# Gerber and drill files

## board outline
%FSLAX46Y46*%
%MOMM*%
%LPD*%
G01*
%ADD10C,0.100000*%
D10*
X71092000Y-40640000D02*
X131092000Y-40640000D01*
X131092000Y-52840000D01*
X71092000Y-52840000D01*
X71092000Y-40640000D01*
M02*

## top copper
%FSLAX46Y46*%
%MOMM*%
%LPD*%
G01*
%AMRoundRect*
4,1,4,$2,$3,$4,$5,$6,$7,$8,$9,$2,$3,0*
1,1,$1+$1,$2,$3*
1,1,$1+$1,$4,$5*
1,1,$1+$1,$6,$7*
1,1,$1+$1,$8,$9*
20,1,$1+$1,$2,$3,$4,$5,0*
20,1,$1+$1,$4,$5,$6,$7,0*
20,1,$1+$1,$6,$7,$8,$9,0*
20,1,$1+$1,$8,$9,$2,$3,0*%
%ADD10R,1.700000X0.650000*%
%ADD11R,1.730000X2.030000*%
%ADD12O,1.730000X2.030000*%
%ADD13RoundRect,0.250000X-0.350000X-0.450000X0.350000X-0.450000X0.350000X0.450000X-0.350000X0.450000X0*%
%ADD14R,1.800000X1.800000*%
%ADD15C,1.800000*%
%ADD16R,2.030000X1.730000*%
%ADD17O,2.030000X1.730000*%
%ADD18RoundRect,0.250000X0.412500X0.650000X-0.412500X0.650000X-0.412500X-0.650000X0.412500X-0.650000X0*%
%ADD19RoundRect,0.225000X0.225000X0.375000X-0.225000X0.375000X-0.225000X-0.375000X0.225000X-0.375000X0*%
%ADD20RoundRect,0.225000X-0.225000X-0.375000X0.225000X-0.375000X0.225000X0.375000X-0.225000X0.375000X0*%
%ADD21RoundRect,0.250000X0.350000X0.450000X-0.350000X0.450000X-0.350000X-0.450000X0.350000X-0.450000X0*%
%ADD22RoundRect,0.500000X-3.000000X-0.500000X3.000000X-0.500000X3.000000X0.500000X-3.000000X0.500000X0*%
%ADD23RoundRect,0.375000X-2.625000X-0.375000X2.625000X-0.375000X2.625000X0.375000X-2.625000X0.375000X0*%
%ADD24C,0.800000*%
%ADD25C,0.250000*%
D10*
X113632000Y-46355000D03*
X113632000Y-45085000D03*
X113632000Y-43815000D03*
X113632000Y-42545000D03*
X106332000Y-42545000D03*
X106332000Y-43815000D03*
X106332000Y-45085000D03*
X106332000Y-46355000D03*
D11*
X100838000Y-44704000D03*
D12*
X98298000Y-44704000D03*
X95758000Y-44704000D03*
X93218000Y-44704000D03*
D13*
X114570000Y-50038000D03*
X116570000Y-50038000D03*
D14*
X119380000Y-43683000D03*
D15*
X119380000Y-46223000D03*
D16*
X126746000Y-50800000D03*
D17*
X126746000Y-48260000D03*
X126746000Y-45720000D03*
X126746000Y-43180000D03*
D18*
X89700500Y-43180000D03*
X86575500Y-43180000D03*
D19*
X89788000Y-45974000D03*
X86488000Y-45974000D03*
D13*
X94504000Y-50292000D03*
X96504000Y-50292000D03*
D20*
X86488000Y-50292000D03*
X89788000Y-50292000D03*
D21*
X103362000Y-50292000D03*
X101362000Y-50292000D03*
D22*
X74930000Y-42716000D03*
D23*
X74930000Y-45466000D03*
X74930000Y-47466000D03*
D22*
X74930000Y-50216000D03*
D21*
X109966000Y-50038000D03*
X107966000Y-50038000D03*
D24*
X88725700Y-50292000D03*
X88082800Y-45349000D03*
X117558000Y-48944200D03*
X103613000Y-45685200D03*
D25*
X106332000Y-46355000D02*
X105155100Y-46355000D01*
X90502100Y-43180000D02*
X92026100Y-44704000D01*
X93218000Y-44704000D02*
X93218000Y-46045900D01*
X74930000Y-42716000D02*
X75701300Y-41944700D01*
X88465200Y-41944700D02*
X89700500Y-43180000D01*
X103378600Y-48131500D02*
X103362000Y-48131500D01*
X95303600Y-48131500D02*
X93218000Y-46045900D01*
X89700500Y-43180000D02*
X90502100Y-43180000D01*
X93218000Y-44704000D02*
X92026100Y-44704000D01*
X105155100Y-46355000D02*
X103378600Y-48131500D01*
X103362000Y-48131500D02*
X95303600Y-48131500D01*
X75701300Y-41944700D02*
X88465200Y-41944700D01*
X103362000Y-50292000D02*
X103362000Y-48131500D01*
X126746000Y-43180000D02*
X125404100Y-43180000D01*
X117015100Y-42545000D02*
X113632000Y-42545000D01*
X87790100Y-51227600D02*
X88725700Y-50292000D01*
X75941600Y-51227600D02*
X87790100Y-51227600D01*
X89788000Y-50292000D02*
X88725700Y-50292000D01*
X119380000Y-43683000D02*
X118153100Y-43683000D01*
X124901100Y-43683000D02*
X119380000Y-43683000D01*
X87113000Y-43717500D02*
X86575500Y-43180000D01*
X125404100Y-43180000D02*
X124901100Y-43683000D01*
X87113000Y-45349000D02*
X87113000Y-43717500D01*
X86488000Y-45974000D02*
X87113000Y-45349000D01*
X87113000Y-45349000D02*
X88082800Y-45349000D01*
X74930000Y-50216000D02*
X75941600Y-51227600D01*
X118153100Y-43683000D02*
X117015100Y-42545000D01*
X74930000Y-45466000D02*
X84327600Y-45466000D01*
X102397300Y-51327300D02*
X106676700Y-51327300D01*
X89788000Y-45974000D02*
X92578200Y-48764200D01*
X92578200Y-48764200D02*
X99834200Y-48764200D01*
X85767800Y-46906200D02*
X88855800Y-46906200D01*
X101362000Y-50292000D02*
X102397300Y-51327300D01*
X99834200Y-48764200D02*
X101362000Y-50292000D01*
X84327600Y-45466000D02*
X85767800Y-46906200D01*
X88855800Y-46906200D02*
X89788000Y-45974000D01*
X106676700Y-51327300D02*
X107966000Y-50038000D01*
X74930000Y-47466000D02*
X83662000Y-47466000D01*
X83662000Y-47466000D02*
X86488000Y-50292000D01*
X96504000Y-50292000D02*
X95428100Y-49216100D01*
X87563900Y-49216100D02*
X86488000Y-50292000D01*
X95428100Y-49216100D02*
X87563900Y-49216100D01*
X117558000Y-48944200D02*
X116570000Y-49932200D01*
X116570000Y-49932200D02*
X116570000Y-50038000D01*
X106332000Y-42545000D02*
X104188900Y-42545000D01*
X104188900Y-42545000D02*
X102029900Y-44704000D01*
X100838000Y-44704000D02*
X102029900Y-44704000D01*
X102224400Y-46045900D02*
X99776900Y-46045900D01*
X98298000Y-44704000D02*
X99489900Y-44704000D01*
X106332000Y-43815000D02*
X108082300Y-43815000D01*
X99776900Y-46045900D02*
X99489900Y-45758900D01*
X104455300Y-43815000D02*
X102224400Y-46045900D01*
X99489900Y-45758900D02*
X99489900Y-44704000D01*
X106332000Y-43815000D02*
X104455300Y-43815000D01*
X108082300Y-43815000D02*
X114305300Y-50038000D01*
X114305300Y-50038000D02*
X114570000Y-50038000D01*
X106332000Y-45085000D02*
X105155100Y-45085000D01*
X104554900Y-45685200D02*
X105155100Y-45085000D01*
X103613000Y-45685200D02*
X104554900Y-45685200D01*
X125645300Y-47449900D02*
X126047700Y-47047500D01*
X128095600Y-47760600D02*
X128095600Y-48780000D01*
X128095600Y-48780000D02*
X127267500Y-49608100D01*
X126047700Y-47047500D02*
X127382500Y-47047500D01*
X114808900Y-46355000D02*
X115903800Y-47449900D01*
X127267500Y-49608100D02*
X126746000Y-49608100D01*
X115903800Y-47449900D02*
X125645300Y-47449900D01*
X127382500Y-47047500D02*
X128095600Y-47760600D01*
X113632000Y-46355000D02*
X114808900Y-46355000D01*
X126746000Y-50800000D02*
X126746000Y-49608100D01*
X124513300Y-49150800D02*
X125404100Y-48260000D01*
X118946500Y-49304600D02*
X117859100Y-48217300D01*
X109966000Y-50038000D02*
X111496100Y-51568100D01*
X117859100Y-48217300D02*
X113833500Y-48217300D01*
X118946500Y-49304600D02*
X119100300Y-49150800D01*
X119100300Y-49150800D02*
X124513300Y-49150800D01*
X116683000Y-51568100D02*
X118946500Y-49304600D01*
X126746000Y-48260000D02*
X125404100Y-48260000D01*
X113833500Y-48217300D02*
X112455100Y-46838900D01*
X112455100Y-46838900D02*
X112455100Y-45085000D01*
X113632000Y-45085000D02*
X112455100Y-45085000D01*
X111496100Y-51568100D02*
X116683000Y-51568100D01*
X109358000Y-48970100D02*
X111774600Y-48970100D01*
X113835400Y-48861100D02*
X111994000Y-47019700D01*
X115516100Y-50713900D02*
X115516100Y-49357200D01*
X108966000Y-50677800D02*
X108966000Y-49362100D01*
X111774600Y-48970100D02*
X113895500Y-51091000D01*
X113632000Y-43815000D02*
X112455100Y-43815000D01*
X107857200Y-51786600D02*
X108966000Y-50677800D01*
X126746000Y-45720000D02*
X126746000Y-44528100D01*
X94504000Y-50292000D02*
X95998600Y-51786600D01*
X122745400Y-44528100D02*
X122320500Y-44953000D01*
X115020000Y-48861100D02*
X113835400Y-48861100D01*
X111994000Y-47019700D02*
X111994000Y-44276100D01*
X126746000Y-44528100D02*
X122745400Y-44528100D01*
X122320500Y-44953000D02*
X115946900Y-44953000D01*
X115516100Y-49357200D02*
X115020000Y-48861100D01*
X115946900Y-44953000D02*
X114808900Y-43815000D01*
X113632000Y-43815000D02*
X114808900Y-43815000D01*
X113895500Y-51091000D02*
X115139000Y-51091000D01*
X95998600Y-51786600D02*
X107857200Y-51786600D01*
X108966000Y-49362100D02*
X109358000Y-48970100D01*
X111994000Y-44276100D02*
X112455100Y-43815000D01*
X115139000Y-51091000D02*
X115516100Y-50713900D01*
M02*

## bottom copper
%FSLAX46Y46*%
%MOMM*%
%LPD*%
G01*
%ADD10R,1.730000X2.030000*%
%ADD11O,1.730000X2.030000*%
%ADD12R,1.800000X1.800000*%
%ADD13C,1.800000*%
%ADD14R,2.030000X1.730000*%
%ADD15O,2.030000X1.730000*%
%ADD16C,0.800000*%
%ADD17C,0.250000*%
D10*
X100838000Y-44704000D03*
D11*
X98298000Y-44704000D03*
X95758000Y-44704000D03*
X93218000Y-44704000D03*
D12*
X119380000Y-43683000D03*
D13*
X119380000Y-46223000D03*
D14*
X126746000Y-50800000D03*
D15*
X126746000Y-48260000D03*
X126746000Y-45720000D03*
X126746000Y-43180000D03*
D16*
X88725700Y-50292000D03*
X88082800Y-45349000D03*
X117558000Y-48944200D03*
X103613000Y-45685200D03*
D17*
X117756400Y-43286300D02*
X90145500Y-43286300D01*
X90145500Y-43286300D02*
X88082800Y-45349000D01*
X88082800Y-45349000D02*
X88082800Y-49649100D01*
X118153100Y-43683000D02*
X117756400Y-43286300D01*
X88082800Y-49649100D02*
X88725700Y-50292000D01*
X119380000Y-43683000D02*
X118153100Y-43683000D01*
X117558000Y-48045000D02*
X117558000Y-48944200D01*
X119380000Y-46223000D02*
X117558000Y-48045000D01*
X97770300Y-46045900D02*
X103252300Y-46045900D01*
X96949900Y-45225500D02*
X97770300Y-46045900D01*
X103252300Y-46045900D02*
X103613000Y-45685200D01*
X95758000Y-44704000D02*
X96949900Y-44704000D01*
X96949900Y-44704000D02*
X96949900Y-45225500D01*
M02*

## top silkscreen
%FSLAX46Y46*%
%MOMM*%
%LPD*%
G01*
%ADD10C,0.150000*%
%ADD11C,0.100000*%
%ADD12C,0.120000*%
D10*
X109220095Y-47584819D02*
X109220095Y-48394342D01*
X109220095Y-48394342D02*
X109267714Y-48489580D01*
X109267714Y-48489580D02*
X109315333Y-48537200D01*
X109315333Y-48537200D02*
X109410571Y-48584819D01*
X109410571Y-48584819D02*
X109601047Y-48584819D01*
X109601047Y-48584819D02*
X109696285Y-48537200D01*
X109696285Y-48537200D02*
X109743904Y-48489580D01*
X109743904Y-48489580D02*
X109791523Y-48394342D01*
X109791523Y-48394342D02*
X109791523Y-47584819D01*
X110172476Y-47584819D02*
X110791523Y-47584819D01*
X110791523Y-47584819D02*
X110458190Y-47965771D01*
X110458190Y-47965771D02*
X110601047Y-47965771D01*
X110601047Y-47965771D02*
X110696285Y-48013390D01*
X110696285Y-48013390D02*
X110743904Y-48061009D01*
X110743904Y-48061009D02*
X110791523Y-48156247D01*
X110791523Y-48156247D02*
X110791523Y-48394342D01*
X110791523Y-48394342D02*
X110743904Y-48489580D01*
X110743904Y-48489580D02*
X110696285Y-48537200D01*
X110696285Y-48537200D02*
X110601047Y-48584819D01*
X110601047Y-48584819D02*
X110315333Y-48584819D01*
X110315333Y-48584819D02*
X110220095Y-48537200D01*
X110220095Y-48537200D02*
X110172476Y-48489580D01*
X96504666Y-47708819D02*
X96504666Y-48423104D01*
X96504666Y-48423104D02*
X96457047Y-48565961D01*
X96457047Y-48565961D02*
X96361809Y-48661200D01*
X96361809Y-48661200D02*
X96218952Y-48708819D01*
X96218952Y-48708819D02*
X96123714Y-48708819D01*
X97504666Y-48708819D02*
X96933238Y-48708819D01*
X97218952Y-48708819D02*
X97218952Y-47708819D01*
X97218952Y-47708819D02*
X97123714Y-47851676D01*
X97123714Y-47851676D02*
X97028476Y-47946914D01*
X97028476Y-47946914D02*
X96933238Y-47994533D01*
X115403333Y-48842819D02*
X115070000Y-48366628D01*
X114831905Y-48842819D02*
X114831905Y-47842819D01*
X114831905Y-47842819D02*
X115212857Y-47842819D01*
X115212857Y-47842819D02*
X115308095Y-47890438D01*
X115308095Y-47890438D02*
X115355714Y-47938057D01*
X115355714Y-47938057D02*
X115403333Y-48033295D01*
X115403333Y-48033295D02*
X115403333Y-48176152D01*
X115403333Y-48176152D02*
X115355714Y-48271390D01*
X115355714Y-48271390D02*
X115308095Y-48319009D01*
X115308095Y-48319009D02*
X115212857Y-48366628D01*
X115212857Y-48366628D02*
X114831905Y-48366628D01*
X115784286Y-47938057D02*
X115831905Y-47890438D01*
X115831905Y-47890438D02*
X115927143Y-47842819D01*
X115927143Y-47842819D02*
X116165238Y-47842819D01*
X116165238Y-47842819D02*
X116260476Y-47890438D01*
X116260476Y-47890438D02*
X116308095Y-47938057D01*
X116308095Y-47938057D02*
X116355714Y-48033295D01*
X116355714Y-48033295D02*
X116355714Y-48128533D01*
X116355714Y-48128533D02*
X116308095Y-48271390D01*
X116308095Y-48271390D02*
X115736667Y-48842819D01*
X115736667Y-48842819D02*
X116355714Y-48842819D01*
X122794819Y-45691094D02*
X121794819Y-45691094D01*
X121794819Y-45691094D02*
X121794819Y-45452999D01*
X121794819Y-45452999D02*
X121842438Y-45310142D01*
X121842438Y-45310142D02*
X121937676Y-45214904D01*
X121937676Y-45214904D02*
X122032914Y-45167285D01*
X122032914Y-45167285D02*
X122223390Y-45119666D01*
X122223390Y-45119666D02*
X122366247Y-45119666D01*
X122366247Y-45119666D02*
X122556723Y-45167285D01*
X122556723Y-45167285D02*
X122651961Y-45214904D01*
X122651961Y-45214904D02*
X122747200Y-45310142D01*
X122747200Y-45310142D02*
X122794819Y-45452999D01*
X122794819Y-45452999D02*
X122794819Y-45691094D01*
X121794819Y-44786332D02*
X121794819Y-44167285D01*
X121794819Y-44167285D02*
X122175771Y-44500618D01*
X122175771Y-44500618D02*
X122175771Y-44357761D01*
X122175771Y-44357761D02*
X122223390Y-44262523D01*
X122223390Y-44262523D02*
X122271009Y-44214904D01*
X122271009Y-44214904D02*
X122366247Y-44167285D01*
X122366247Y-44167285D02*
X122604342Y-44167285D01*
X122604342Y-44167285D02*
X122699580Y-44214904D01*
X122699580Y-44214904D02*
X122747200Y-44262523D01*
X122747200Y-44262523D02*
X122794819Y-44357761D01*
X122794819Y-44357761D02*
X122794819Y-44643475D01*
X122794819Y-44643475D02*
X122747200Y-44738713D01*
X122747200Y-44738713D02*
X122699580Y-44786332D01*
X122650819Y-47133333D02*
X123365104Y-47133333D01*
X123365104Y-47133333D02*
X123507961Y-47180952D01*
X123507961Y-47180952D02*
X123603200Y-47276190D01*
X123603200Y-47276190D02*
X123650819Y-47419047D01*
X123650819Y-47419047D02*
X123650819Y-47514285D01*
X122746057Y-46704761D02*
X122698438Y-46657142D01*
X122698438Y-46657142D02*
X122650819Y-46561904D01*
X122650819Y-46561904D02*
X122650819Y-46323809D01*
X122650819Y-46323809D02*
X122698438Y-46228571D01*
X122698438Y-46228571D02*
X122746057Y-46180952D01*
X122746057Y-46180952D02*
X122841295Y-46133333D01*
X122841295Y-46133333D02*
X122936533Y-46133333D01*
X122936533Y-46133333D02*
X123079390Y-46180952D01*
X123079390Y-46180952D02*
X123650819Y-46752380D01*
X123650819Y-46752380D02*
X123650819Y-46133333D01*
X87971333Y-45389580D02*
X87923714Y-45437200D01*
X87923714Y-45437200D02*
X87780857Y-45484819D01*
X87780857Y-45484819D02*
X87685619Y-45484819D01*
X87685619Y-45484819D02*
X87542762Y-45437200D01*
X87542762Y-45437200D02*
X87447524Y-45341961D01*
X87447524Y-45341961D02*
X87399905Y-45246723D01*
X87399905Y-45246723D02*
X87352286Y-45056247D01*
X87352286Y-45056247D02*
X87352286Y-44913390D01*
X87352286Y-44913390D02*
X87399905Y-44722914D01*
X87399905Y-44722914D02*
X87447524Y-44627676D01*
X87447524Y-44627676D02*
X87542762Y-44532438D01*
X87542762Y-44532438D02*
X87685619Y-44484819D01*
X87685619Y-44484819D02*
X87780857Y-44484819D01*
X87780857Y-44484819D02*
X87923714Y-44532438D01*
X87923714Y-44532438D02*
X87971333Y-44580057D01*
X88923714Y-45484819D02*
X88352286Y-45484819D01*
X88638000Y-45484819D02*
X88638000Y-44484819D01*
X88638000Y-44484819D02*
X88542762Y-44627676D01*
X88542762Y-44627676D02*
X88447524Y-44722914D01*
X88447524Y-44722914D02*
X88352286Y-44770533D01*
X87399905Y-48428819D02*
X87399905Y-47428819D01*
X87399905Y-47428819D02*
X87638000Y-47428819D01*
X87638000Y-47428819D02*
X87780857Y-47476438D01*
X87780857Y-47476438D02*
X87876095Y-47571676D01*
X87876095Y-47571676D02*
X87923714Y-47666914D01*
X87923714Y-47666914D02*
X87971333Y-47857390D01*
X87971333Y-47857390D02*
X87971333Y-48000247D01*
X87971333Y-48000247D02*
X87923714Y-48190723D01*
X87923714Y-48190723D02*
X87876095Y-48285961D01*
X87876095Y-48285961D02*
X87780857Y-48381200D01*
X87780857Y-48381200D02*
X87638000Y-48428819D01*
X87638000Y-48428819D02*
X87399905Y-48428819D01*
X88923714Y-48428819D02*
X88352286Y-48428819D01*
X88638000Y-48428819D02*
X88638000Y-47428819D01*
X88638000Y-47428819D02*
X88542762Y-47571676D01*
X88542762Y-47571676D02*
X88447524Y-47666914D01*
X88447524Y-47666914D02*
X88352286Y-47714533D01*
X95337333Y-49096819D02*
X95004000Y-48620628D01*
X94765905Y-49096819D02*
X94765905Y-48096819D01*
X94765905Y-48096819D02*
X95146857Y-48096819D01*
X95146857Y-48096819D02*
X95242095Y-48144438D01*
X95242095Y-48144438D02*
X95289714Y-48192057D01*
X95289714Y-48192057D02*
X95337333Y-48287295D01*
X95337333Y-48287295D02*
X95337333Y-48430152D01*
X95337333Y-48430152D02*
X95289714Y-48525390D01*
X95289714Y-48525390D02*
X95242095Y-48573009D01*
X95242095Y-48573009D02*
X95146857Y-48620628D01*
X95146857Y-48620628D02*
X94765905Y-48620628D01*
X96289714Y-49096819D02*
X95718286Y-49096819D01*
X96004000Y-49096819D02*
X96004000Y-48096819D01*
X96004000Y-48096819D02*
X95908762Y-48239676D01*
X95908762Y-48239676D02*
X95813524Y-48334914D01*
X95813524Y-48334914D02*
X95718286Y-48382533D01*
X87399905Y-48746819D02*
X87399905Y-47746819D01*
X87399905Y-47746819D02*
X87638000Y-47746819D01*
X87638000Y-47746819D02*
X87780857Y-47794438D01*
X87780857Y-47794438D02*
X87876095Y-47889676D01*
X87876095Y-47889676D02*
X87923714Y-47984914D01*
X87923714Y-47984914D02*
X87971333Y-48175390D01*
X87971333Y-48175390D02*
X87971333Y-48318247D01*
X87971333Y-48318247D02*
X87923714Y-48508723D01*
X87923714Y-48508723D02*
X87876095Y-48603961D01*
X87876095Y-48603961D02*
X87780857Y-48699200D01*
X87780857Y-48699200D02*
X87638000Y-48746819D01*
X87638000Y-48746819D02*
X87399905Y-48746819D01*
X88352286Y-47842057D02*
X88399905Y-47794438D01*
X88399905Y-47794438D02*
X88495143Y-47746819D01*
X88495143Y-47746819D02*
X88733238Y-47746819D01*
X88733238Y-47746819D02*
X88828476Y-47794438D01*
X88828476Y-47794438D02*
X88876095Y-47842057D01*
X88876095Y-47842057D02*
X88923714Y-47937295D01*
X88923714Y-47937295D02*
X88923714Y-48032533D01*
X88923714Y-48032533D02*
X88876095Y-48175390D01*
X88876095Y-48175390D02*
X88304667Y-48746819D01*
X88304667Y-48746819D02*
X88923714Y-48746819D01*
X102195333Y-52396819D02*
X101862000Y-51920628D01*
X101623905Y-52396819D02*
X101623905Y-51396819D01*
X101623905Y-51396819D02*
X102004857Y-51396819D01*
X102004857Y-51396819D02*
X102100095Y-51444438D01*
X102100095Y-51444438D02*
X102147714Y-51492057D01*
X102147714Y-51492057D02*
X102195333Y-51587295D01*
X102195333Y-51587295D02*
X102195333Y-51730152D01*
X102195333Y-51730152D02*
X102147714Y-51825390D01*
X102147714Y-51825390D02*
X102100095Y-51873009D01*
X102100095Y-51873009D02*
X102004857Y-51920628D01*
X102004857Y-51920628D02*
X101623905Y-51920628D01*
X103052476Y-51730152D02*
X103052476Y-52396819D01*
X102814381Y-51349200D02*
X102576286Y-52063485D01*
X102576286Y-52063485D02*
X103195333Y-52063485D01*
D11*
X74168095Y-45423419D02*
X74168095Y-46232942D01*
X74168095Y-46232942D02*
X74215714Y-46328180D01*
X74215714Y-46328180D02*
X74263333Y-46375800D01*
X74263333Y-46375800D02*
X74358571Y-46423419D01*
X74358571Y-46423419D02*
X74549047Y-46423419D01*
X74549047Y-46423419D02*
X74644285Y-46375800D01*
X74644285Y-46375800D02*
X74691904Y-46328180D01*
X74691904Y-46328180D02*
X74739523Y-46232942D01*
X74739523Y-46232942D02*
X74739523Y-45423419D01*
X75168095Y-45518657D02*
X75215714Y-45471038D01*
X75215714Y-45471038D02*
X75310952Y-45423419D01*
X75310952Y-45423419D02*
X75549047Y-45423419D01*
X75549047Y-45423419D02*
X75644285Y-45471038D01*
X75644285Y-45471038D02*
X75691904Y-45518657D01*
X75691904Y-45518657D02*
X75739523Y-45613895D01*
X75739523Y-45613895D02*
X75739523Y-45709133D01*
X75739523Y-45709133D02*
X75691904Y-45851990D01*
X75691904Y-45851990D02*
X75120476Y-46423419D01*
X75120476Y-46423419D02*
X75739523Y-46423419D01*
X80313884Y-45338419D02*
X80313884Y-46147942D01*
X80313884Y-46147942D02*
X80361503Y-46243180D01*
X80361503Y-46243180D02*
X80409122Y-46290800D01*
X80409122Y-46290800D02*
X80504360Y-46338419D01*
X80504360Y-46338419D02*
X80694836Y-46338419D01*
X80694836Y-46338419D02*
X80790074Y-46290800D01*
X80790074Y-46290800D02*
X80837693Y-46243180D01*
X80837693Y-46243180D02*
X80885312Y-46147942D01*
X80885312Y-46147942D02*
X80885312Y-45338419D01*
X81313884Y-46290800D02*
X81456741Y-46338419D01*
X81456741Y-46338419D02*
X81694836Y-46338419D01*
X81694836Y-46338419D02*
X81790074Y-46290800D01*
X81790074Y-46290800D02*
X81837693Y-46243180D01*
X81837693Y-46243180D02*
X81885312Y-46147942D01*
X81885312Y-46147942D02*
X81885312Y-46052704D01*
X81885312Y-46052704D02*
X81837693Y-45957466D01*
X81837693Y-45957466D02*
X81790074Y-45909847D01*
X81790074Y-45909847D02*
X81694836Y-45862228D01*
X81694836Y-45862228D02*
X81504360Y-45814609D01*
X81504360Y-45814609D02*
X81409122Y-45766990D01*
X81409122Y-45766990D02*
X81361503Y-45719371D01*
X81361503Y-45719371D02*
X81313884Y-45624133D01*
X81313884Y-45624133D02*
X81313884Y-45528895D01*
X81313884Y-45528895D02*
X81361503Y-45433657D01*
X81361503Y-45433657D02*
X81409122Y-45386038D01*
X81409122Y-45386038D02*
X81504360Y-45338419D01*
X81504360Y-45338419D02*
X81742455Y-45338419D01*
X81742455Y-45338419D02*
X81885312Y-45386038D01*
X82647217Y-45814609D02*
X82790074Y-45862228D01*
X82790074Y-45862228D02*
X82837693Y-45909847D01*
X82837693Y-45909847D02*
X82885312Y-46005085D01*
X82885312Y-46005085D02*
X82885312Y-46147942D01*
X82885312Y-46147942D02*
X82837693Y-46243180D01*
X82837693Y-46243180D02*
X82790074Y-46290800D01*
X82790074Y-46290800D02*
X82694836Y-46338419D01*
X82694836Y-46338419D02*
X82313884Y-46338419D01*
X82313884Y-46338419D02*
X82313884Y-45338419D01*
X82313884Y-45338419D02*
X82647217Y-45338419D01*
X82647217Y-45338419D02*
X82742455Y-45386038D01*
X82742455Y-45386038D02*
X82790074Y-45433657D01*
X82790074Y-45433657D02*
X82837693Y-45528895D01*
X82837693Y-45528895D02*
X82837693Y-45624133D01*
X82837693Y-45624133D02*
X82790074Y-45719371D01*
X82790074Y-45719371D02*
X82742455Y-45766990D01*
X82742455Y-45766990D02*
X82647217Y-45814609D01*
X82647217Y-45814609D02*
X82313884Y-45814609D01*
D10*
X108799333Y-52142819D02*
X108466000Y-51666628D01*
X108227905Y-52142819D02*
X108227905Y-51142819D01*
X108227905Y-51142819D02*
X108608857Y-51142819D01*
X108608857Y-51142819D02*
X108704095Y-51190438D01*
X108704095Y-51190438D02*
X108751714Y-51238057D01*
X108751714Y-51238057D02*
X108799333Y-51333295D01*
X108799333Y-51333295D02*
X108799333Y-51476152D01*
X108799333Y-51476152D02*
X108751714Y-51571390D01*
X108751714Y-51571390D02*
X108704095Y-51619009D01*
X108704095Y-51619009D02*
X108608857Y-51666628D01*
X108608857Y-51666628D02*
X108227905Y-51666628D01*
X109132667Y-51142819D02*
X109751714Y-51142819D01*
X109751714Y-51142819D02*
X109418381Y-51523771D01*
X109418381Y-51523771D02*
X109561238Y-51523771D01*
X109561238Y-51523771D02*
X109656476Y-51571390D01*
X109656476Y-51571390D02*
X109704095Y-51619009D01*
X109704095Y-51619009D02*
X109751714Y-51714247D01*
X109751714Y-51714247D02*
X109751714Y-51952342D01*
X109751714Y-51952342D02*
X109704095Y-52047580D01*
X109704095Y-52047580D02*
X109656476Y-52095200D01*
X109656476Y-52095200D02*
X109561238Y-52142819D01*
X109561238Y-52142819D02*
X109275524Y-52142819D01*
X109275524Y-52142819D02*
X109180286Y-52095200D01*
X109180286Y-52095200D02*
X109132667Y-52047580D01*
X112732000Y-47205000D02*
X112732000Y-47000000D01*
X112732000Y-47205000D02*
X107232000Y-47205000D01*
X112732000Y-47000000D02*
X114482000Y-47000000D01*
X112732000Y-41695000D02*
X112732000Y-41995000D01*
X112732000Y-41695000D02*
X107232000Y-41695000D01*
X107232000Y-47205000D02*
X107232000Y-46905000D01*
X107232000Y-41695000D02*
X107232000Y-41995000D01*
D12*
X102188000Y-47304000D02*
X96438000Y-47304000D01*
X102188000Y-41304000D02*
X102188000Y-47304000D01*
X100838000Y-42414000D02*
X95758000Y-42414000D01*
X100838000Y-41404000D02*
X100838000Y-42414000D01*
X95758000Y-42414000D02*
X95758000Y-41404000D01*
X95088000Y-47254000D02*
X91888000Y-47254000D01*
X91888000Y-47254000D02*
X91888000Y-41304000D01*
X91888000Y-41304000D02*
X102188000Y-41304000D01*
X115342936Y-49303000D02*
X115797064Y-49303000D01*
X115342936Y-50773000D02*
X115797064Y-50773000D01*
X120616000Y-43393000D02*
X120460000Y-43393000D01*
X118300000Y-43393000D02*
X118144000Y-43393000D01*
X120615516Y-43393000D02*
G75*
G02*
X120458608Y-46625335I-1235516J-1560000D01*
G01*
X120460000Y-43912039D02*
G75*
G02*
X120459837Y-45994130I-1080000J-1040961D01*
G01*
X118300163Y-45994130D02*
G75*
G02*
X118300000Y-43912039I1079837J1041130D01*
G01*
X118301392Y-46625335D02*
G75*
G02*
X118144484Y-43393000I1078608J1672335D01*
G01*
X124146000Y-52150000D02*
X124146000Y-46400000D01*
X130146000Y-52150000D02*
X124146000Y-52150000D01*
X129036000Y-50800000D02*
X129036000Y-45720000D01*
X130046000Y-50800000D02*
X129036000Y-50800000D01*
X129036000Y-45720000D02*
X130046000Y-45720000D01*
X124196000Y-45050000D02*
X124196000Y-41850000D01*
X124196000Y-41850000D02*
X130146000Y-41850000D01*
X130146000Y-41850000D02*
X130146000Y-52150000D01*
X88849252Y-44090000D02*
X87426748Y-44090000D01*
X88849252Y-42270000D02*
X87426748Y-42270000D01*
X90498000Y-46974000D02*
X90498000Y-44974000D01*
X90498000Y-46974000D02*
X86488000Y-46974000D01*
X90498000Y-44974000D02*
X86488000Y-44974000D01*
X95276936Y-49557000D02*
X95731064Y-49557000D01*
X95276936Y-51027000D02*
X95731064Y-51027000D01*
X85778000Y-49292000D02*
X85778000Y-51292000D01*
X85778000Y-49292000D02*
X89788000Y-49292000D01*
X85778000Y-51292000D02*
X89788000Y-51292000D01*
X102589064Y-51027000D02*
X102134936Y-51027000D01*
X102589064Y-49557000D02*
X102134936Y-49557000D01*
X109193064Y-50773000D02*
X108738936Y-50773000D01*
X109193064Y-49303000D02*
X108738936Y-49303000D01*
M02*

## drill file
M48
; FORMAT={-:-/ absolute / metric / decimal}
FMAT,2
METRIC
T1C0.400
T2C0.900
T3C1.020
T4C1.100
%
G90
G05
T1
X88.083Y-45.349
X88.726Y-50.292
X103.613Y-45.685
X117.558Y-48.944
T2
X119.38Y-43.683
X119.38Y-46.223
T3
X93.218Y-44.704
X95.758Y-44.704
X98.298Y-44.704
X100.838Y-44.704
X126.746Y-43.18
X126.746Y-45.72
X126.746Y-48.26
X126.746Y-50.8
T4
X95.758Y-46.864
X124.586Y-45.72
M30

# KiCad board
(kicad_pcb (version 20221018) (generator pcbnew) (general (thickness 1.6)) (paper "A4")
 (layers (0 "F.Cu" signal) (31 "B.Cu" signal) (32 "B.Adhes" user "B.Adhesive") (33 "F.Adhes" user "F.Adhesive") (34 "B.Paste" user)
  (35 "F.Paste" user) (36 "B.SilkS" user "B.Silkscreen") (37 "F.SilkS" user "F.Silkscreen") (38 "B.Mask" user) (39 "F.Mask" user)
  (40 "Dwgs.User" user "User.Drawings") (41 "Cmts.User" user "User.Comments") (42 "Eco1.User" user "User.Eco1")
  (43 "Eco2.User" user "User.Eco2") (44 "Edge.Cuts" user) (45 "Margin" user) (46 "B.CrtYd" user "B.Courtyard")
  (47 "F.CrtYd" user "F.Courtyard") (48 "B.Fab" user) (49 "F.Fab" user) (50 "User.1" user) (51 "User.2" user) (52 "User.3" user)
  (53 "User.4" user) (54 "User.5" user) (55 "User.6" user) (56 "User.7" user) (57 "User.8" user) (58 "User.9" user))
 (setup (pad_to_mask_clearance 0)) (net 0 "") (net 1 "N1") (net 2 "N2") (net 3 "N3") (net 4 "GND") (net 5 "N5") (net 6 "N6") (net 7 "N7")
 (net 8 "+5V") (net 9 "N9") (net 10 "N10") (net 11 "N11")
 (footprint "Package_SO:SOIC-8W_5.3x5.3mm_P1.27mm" (layer "F.Cu") (at 109.982 44.45 180)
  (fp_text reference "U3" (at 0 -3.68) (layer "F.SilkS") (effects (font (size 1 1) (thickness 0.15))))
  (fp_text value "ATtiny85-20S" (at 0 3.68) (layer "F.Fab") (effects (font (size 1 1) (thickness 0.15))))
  (fp_line (start -2.75 -2.755) (end -2.75 -2.55) (stroke (width 0.15) (type solid)) (layer "F.SilkS"))
  (fp_line (start -2.75 -2.755) (end 2.75 -2.755) (stroke (width 0.15) (type solid)) (layer "F.SilkS"))
  (fp_line (start -2.75 -2.55) (end -4.5 -2.55) (stroke (width 0.15) (type solid)) (layer "F.SilkS"))
  (fp_line (start -2.75 2.755) (end -2.75 2.455) (stroke (width 0.15) (type solid)) (layer "F.SilkS"))
  (fp_line (start -2.75 2.755) (end 2.75 2.755) (stroke (width 0.15) (type solid)) (layer "F.SilkS"))
  (fp_line (start 2.75 -2.755) (end 2.75 -2.455) (stroke (width 0.15) (type solid)) (layer "F.SilkS"))
  (fp_line (start 2.75 2.755) (end 2.75 2.455) (stroke (width 0.15) (type solid)) (layer "F.SilkS"))
  (pad "1" smd rect (at -3.65 -1.905 180) (size 1.7 0.65) (layers "F.Cu" "F.Paste" "F.Mask") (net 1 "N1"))
  (pad "2" smd rect (at -3.65 -0.635 180) (size 1.7 0.65) (layers "F.Cu" "F.Paste" "F.Mask") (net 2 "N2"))
  (pad "3" smd rect (at -3.65 0.635 180) (size 1.7 0.65) (layers "F.Cu" "F.Paste" "F.Mask") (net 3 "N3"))
  (pad "4" smd rect (at -3.65 1.905 180) (size 1.7 0.65) (layers "F.Cu" "F.Paste" "F.Mask") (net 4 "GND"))
  (pad "5" smd rect (at 3.65 1.905 180) (size 1.7 0.65) (layers "F.Cu" "F.Paste" "F.Mask") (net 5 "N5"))
  (pad "6" smd rect (at 3.65 0.635 180) (size 1.7 0.65) (layers "F.Cu" "F.Paste" "F.Mask") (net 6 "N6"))
  (pad "7" smd rect (at 3.65 -0.635 180) (size 1.7 0.65) (layers "F.Cu" "F.Paste" "F.Mask") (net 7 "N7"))
  (pad "8" smd rect (at 3.65 -1.905 180) (size 1.7 0.65) (layers "F.Cu" "F.Paste" "F.Mask") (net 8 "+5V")))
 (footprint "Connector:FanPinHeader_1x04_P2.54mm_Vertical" (layer "F.Cu") (at 100.838 44.704 180)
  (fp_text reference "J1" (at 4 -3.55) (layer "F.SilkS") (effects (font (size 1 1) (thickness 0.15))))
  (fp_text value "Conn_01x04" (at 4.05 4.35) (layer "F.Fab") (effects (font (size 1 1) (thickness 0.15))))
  (fp_line (start -1.35 -2.6) (end 4.4 -2.6) (stroke (width 0.12) (type solid)) (layer "F.SilkS"))
  (fp_line (start -1.35 3.4) (end -1.35 -2.6) (stroke (width 0.12) (type solid)) (layer "F.SilkS"))
  (fp_line (start 0 2.29) (end 5.08 2.29) (stroke (width 0.12) (type solid)) (layer "F.SilkS"))
  (fp_line (start 0 3.3) (end 0 2.29) (stroke (width 0.12) (type solid)) (layer "F.SilkS"))
  (fp_line (start 5.08 2.29) (end 5.08 3.3) (stroke (width 0.12) (type solid)) (layer "F.SilkS"))
  (fp_line (start 5.75 -2.55) (end 8.95 -2.55) (stroke (width 0.12) (type solid)) (layer "F.SilkS"))
  (fp_line (start 8.95 -2.55) (end 8.95 3.4) (stroke (width 0.12) (type solid)) (layer "F.SilkS"))
  (fp_line (start 8.95 3.4) (end -1.35 3.4) (stroke (width 0.12) (type solid)) (layer "F.SilkS"))
  (pad "" np_thru_hole circle (at 5.08 -2.16 270) (size 1.1 1.1) (drill 1.1) (layers "*.Cu" "*.Mask"))
  (pad "1" thru_hole rect (at 0 0 270) (size 2.03 1.73) (drill 1.02) (layers "*.Cu" "*.Mask") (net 5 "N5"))
  (pad "2" thru_hole oval (at 2.54 0 270) (size 2.03 1.73) (drill 1.02) (layers "*.Cu" "*.Mask") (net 6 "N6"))
  (pad "3" thru_hole oval (at 5.08 0 270) (size 2.03 1.73) (drill 1.02) (layers "*.Cu" "*.Mask") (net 7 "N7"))
  (pad "4" thru_hole oval (at 7.62 0 270) (size 2.03 1.73) (drill 1.02) (layers "*.Cu" "*.Mask") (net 8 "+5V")))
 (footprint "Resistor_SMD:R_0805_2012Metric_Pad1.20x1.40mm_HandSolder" (layer "F.Cu") (at 115.57 50.038)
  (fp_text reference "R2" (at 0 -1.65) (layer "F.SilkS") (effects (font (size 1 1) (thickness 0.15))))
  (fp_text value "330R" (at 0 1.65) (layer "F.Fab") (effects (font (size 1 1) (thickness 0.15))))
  (fp_line (start -0.227064 -0.735) (end 0.227064 -0.735) (stroke (width 0.12) (type solid)) (layer "F.SilkS"))
  (fp_line (start -0.227064 0.735) (end 0.227064 0.735) (stroke (width 0.12) (type solid)) (layer "F.SilkS"))
  (pad "1" smd roundrect (at -1 0) (size 1.2 1.4) (layers "F.Cu" "F.Paste" "F.Mask") (roundrect_rratio 0.208333) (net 6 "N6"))
  (pad "2" smd roundrect (at 1 0) (size 1.2 1.4) (layers "F.Cu" "F.Paste" "F.Mask") (roundrect_rratio 0.208333) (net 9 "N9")))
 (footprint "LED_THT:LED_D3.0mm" (layer "F.Cu") (at 119.38 43.683 -90)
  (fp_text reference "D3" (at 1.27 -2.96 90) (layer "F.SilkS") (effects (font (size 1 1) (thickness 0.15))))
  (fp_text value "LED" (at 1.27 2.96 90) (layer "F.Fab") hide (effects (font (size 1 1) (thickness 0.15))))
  (fp_line (start -0.29 -1.236) (end -0.29 -1.08) (stroke (width 0.12) (type solid)) (layer "F.SilkS"))
  (fp_line (start -0.29 1.08) (end -0.29 1.236) (stroke (width 0.12) (type solid)) (layer "F.SilkS"))
  (fp_arc (start -0.29 -1.235516) (mid 1.366487 -1.987659) (end 2.942335 -1.078608) (stroke (width 0.12) (type solid)) (layer "F.SilkS"))
  (fp_arc (start 0.229039 -1.08) (mid 1.270117 -1.5) (end 2.31113 -1.079837) (stroke (width 0.12) (type solid)) (layer "F.SilkS"))
  (fp_arc (start 2.31113 1.079837) (mid 1.270117 1.5) (end 0.229039 1.08) (stroke (width 0.12) (type solid)) (layer "F.SilkS"))
  (fp_arc (start 2.942335 1.078608) (mid 1.366487 1.987659) (end -0.29 1.235516) (stroke (width 0.12) (type solid)) (layer "F.SilkS"))
  (pad "1" thru_hole rect (at 0 0 270) (size 1.8 1.8) (drill 0.9) (layers "*.Cu" "*.Mask") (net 4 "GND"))
  (pad "2" thru_hole circle (at 2.54 0 270) (size 1.8 1.8) (drill 0.9) (layers "*.Cu" "*.Mask") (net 9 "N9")))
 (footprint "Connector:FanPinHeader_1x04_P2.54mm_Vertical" (layer "F.Cu") (at 126.746 50.8 90)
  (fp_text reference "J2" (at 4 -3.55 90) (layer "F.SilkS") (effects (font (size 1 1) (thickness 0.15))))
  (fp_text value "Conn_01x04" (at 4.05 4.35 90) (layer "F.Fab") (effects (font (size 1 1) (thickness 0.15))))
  (fp_line (start -1.35 -2.6) (end 4.4 -2.6) (stroke (width 0.12) (type solid)) (layer "F.SilkS"))
  (fp_line (start -1.35 3.4) (end -1.35 -2.6) (stroke (width 0.12) (type solid)) (layer "F.SilkS"))
  (fp_line (start 0 2.29) (end 5.08 2.29) (stroke (width 0.12) (type solid)) (layer "F.SilkS"))
  (fp_line (start 0 3.3) (end 0 2.29) (stroke (width 0.12) (type solid)) (layer "F.SilkS"))
  (fp_line (start 5.08 2.29) (end 5.08 3.3) (stroke (width 0.12) (type solid)) (layer "F.SilkS"))
  (fp_line (start 5.75 -2.55) (end 8.95 -2.55) (stroke (width 0.12) (type solid)) (layer "F.SilkS"))
  (fp_line (start 8.95 -2.55) (end 8.95 3.4) (stroke (width 0.12) (type solid)) (layer "F.SilkS"))
  (fp_line (start 8.95 3.4) (end -1.35 3.4) (stroke (width 0.12) (type solid)) (layer "F.SilkS"))
  (pad "" np_thru_hole circle (at 5.08 -2.16 180) (size 1.1 1.1) (drill 1.1) (layers "*.Cu" "*.Mask"))
  (pad "1" thru_hole rect (at 0 0 180) (size 2.03 1.73) (drill 1.02) (layers "*.Cu" "*.Mask") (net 1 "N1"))
  (pad "2" thru_hole oval (at 2.54 0 180) (size 2.03 1.73) (drill 1.02) (layers "*.Cu" "*.Mask") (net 2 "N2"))
  (pad "3" thru_hole oval (at 5.08 0 180) (size 2.03 1.73) (drill 1.02) (layers "*.Cu" "*.Mask") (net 3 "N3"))
  (pad "4" thru_hole oval (at 7.62 0 180) (size 2.03 1.73) (drill 1.02) (layers "*.Cu" "*.Mask") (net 4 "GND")))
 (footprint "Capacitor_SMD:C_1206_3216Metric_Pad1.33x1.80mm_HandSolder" (layer "F.Cu") (at 88.138 43.18 180)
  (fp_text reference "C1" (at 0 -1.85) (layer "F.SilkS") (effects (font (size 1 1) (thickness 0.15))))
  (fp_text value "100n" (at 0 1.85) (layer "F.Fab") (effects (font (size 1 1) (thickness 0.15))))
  (fp_line (start -0.711252 -0.91) (end 0.711252 -0.91) (stroke (width 0.12) (type solid)) (layer "F.SilkS"))
  (fp_line (start -0.711252 0.91) (end 0.711252 0.91) (stroke (width 0.12) (type solid)) (layer "F.SilkS"))
  (pad "1" smd roundrect (at -1.5625 0 180) (size 1.325 1.8) (layers "F.Cu" "F.Paste" "F.Mask") (roundrect_rratio 0.188679) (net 8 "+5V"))
  (pad "2" smd roundrect (at 1.5625 0 180) (size 1.325 1.8) (layers "F.Cu" "F.Paste" "F.Mask") (roundrect_rratio 0.188679) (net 4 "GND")))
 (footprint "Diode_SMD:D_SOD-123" (layer "F.Cu") (at 88.138 45.974 180)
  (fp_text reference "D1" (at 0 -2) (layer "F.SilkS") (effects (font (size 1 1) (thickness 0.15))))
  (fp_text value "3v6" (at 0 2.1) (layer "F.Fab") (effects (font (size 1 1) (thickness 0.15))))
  (fp_line (start -2.36 -1) (end -2.36 1) (stroke (width 0.12) (type solid)) (layer "F.SilkS"))
  (fp_line (start -2.36 -1) (end 1.65 -1) (stroke (width 0.12) (type solid)) (layer "F.SilkS"))
  (fp_line (start -2.36 1) (end 1.65 1) (stroke (width 0.12) (type solid)) (layer "F.SilkS"))
  (pad "1" smd roundrect (at -1.65 0 180) (size 0.9 1.2) (layers "F.Cu" "F.Paste" "F.Mask") (roundrect_rratio 0.25) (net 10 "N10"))
  (pad "2" smd roundrect (at 1.65 0 180) (size 0.9 1.2) (layers "F.Cu" "F.Paste" "F.Mask") (roundrect_rratio 0.25) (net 4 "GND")))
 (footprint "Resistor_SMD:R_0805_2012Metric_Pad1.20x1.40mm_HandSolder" (layer "F.Cu") (at 95.504 50.292)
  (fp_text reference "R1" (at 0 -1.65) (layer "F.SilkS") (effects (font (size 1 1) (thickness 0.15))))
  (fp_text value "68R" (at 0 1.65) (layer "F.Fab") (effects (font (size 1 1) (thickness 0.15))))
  (fp_line (start -0.227064 -0.735) (end 0.227064 -0.735) (stroke (width 0.12) (type solid)) (layer "F.SilkS"))
  (fp_line (start -0.227064 0.735) (end 0.227064 0.735) (stroke (width 0.12) (type solid)) (layer "F.SilkS"))
  (pad "1" smd roundrect (at -1 0) (size 1.2 1.4) (layers "F.Cu" "F.Paste" "F.Mask") (roundrect_rratio 0.208333) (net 3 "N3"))
  (pad "2" smd roundrect (at 1 0) (size 1.2 1.4) (layers "F.Cu" "F.Paste" "F.Mask") (roundrect_rratio 0.208333) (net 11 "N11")))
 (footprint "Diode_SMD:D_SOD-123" (layer "F.Cu") (at 88.138 50.292)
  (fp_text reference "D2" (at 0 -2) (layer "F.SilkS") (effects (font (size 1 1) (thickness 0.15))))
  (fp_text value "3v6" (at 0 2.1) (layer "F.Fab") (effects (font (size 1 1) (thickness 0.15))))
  (fp_line (start -2.36 -1) (end -2.36 1) (stroke (width 0.12) (type solid)) (layer "F.SilkS"))
  (fp_line (start -2.36 -1) (end 1.65 -1) (stroke (width 0.12) (type solid)) (layer "F.SilkS"))
  (fp_line (start -2.36 1) (end 1.65 1) (stroke (width 0.12) (type solid)) (layer "F.SilkS"))
  (pad "1" smd roundrect (at -1.65 0) (size 0.9 1.2) (layers "F.Cu" "F.Paste" "F.Mask") (roundrect_rratio 0.25) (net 11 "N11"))
  (pad "2" smd roundrect (at 1.65 0) (size 0.9 1.2) (layers "F.Cu" "F.Paste" "F.Mask") (roundrect_rratio 0.25) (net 4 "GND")))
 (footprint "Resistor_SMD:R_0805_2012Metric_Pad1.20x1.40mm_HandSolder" (layer "F.Cu") (at 102.362 50.292 180)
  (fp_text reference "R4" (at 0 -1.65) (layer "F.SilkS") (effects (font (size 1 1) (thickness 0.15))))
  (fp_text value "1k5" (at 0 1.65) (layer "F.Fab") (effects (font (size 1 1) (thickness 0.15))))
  (fp_line (start -0.227064 -0.735) (end 0.227064 -0.735) (stroke (width 0.12) (type solid)) (layer "F.SilkS"))
  (fp_line (start -0.227064 0.735) (end 0.227064 0.735) (stroke (width 0.12) (type solid)) (layer "F.SilkS"))
  (pad "1" smd roundrect (at -1 0 180) (size 1.2 1.4) (layers "F.Cu" "F.Paste" "F.Mask") (roundrect_rratio 0.208333) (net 8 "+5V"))
  (pad "2" smd roundrect (at 1 0 180) (size 1.2 1.4) (layers "F.Cu" "F.Paste" "F.Mask") (roundrect_rratio 0.208333) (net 10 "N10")))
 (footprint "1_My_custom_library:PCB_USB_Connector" (layer "F.Cu") (at 74.93 46.466)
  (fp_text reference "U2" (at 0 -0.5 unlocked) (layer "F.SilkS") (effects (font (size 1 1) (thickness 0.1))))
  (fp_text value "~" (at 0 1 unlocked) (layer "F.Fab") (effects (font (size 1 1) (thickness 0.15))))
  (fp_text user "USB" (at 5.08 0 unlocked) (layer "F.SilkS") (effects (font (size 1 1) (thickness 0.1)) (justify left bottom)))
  (pad "1" smd roundrect (at 0 -3.75) (size 7 2) (layers "F.Cu" "F.Paste" "F.Mask") (roundrect_rratio 0.25) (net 8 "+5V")
   (thermal_bridge_angle 45))
  (pad "2" smd roundrect (at 0 -1) (size 6 1.5) (layers "F.Cu" "F.Paste" "F.Mask") (roundrect_rratio 0.25) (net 10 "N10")
   (thermal_bridge_angle 45))
  (pad "3" smd roundrect (at 0 1) (size 6 1.5) (layers "F.Cu" "F.Paste" "F.Mask") (roundrect_rratio 0.25) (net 11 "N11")
   (thermal_bridge_angle 45))
  (pad "4" smd roundrect (at 0 3.75) (size 7 2) (layers "F.Cu" "F.Paste" "F.Mask") (roundrect_rratio 0.25) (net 4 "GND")
   (thermal_bridge_angle 45))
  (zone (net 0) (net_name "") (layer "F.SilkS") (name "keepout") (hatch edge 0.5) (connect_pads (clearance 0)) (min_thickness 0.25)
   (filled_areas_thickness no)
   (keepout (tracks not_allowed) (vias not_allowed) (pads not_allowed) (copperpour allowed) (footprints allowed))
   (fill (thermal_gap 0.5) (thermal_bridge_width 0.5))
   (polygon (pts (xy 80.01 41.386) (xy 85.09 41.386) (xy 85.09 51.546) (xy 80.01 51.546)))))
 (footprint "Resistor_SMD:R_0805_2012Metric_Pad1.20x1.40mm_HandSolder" (layer "F.Cu") (at 108.966 50.038 180)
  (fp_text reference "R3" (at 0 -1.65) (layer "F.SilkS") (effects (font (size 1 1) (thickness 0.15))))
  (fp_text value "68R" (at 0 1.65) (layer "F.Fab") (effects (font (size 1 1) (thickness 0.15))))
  (fp_line (start -0.227064 -0.735) (end 0.227064 -0.735) (stroke (width 0.12) (type solid)) (layer "F.SilkS"))
  (fp_line (start -0.227064 0.735) (end 0.227064 0.735) (stroke (width 0.12) (type solid)) (layer "F.SilkS"))
  (pad "1" smd roundrect (at -1 0 180) (size 1.2 1.4) (layers "F.Cu" "F.Paste" "F.Mask") (roundrect_rratio 0.208333) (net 2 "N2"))
  (pad "2" smd roundrect (at 1 0 180) (size 1.2 1.4) (layers "F.Cu" "F.Paste" "F.Mask") (roundrect_rratio 0.208333) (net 10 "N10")))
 (gr_rect (start 71.092 40.64) (end 131.092 52.84) (stroke (width 0.1) (type default)) (fill none) (layer "Edge.Cuts"))
 (segment (start 106.332 46.355) (end 105.1551 46.355) (width 0.25) (layer "F.Cu") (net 8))
 (segment (start 90.5021 43.18) (end 92.0261 44.704) (width 0.25) (layer "F.Cu") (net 8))
 (segment (start 93.218 44.704) (end 93.218 46.0459) (width 0.25) (layer "F.Cu") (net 8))
 (segment (start 74.93 42.716) (end 75.7013 41.9447) (width 0.25) (layer "F.Cu") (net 8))
 (segment (start 88.4652 41.9447) (end 89.7005 43.18) (width 0.25) (layer "F.Cu") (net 8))
 (segment (start 103.3786 48.1315) (end 103.362 48.1315) (width 0.25) (layer "F.Cu") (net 8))
 (segment (start 95.3036 48.1315) (end 93.218 46.0459) (width 0.25) (layer "F.Cu") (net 8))
 (segment (start 89.7005 43.18) (end 90.5021 43.18) (width 0.25) (layer "F.Cu") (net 8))
 (segment (start 93.218 44.704) (end 92.0261 44.704) (width 0.25) (layer "F.Cu") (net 8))
 (segment (start 105.1551 46.355) (end 103.3786 48.1315) (width 0.25) (layer "F.Cu") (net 8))
 (segment (start 103.362 48.1315) (end 95.3036 48.1315) (width 0.25) (layer "F.Cu") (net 8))
 (segment (start 75.7013 41.9447) (end 88.4652 41.9447) (width 0.25) (layer "F.Cu") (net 8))
 (segment (start 103.362 50.292) (end 103.362 48.1315) (width 0.25) (layer "F.Cu") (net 8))
 (segment (start 126.746 43.18) (end 125.4041 43.18) (width 0.25) (layer "F.Cu") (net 4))
 (segment (start 117.0151 42.545) (end 113.632 42.545) (width 0.25) (layer "F.Cu") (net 4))
 (segment (start 87.7901 51.2276) (end 88.7257 50.292) (width 0.25) (layer "F.Cu") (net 4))
 (segment (start 75.9416 51.2276) (end 87.7901 51.2276) (width 0.25) (layer "F.Cu") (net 4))
 (segment (start 89.788 50.292) (end 88.7257 50.292) (width 0.25) (layer "F.Cu") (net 4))
 (segment (start 119.38 43.683) (end 118.1531 43.683) (width 0.25) (layer "F.Cu") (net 4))
 (segment (start 124.9011 43.683) (end 119.38 43.683) (width 0.25) (layer "F.Cu") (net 4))
 (segment (start 87.113 43.7175) (end 86.5755 43.18) (width 0.25) (layer "F.Cu") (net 4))
 (segment (start 125.4041 43.18) (end 124.9011 43.683) (width 0.25) (layer "F.Cu") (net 4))
 (segment (start 87.113 45.349) (end 87.113 43.7175) (width 0.25) (layer "F.Cu") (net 4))
 (segment (start 86.488 45.974) (end 87.113 45.349) (width 0.25) (layer "F.Cu") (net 4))
 (segment (start 87.113 45.349) (end 88.0828 45.349) (width 0.25) (layer "F.Cu") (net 4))
 (segment (start 74.93 50.216) (end 75.9416 51.2276) (width 0.25) (layer "F.Cu") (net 4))
 (segment (start 118.1531 43.683) (end 117.0151 42.545) (width 0.25) (layer "F.Cu") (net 4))
 (via (at 88.7257 50.292) (size 0.8) (drill 0.4) (layers "F.Cu" "B.Cu") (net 4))
 (via (at 88.0828 45.349) (size 0.8) (drill 0.4) (layers "F.Cu" "B.Cu") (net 4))
 (segment (start 117.7564 43.2863) (end 90.1455 43.2863) (width 0.25) (layer "B.Cu") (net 4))
 (segment (start 90.1455 43.2863) (end 88.0828 45.349) (width 0.25) (layer "B.Cu") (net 4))
 (segment (start 88.0828 45.349) (end 88.0828 49.6491) (width 0.25) (layer "B.Cu") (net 4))
 (segment (start 118.1531 43.683) (end 117.7564 43.2863) (width 0.25) (layer "B.Cu") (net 4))
 (segment (start 88.0828 49.6491) (end 88.7257 50.292) (width 0.25) (layer "B.Cu") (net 4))
 (segment (start 119.38 43.683) (end 118.1531 43.683) (width 0.25) (layer "B.Cu") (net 4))
 (segment (start 74.93 45.466) (end 84.3276 45.466) (width 0.25) (layer "F.Cu") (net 10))
 (segment (start 102.3973 51.3273) (end 106.6767 51.3273) (width 0.25) (layer "F.Cu") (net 10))
 (segment (start 89.788 45.974) (end 92.5782 48.7642) (width 0.25) (layer "F.Cu") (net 10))
 (segment (start 92.5782 48.7642) (end 99.8342 48.7642) (width 0.25) (layer "F.Cu") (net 10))
 (segment (start 85.7678 46.9062) (end 88.8558 46.9062) (width 0.25) (layer "F.Cu") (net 10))
 (segment (start 101.362 50.292) (end 102.3973 51.3273) (width 0.25) (layer "F.Cu") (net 10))
 (segment (start 99.8342 48.7642) (end 101.362 50.292) (width 0.25) (layer "F.Cu") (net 10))
 (segment (start 84.3276 45.466) (end 85.7678 46.9062) (width 0.25) (layer "F.Cu") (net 10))
 (segment (start 88.8558 46.9062) (end 89.788 45.974) (width 0.25) (layer "F.Cu") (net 10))
 (segment (start 106.6767 51.3273) (end 107.966 50.038) (width 0.25) (layer "F.Cu") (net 10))
 (segment (start 74.93 47.466) (end 83.662 47.466) (width 0.25) (layer "F.Cu") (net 11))
 (segment (start 83.662 47.466) (end 86.488 50.292) (width 0.25) (layer "F.Cu") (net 11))
 (segment (start 96.504 50.292) (end 95.4281 49.2161) (width 0.25) (layer "F.Cu") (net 11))
 (segment (start 87.5639 49.2161) (end 86.488 50.292) (width 0.25) (layer "F.Cu") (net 11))
 (segment (start 95.4281 49.2161) (end 87.5639 49.2161) (width 0.25) (layer "F.Cu") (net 11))
 (segment (start 117.558 48.9442) (end 116.57 49.9322) (width 0.25) (layer "F.Cu") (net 9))
 (segment (start 116.57 49.9322) (end 116.57 50.038) (width 0.25) (layer "F.Cu") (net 9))
 (via (at 117.558 48.9442) (size 0.8) (drill 0.4) (layers "F.Cu" "B.Cu") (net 9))
 (segment (start 117.558 48.045) (end 117.558 48.9442) (width 0.25) (layer "B.Cu") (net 9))
 (segment (start 119.38 46.223) (end 117.558 48.045) (width 0.25) (layer "B.Cu") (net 9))
 (segment (start 106.332 42.545) (end 104.1889 42.545) (width 0.25) (layer "F.Cu") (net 5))
 (segment (start 104.1889 42.545) (end 102.0299 44.704) (width 0.25) (layer "F.Cu") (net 5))
 (segment (start 100.838 44.704) (end 102.0299 44.704) (width 0.25) (layer "F.Cu") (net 5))
 (segment (start 102.2244 46.0459) (end 99.7769 46.0459) (width 0.25) (layer "F.Cu") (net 6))
 (segment (start 98.298 44.704) (end 99.4899 44.704) (width 0.25) (layer "F.Cu") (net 6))
 (segment (start 106.332 43.815) (end 108.0823 43.815) (width 0.25) (layer "F.Cu") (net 6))
 (segment (start 99.7769 46.0459) (end 99.4899 45.7589) (width 0.25) (layer "F.Cu") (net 6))
 (segment (start 104.4553 43.815) (end 102.2244 46.0459) (width 0.25) (layer "F.Cu") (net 6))
 (segment (start 99.4899 45.7589) (end 99.4899 44.704) (width 0.25) (layer "F.Cu") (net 6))
 (segment (start 106.332 43.815) (end 104.4553 43.815) (width 0.25) (layer "F.Cu") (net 6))
 (segment (start 108.0823 43.815) (end 114.3053 50.038) (width 0.25) (layer "F.Cu") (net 6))
 (segment (start 114.3053 50.038) (end 114.57 50.038) (width 0.25) (layer "F.Cu") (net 6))
 (segment (start 106.332 45.085) (end 105.1551 45.085) (width 0.25) (layer "F.Cu") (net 7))
 (segment (start 104.5549 45.6852) (end 105.1551 45.085) (width 0.25) (layer "F.Cu") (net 7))
 (segment (start 103.613 45.6852) (end 104.5549 45.6852) (width 0.25) (layer "F.Cu") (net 7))
 (via (at 103.613 45.6852) (size 0.8) (drill 0.4) (layers "F.Cu" "B.Cu") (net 7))
 (segment (start 97.7703 46.0459) (end 103.2523 46.0459) (width 0.25) (layer "B.Cu") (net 7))
 (segment (start 96.9499 45.2255) (end 97.7703 46.0459) (width 0.25) (layer "B.Cu") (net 7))
 (segment (start 103.2523 46.0459) (end 103.613 45.6852) (width 0.25) (layer "B.Cu") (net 7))
 (segment (start 95.758 44.704) (end 96.9499 44.704) (width 0.25) (layer "B.Cu") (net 7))
 (segment (start 96.9499 44.704) (end 96.9499 45.2255) (width 0.25) (layer "B.Cu") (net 7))
 (segment (start 125.6453 47.4499) (end 126.0477 47.0475) (width 0.25) (layer "F.Cu") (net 1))
 (segment (start 128.0956 47.7606) (end 128.0956 48.78) (width 0.25) (layer "F.Cu") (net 1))
 (segment (start 128.0956 48.78) (end 127.2675 49.6081) (width 0.25) (layer "F.Cu") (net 1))
 (segment (start 126.0477 47.0475) (end 127.3825 47.0475) (width 0.25) (layer "F.Cu") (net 1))
 (segment (start 114.8089 46.355) (end 115.9038 47.4499) (width 0.25) (layer "F.Cu") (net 1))
 (segment (start 127.2675 49.6081) (end 126.746 49.6081) (width 0.25) (layer "F.Cu") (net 1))
 (segment (start 115.9038 47.4499) (end 125.6453 47.4499) (width 0.25) (layer "F.Cu") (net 1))
 (segment (start 127.3825 47.0475) (end 128.0956 47.7606) (width 0.25) (layer "F.Cu") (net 1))
 (segment (start 113.632 46.355) (end 114.8089 46.355) (width 0.25) (layer "F.Cu") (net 1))
 (segment (start 126.746 50.8) (end 126.746 49.6081) (width 0.25) (layer "F.Cu") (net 1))
 (segment (start 124.5133 49.1508) (end 125.4041 48.26) (width 0.25) (layer "F.Cu") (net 2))
 (segment (start 118.9465 49.3046) (end 117.8591 48.2173) (width 0.25) (layer "F.Cu") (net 2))
 (segment (start 109.966 50.038) (end 111.4961 51.5681) (width 0.25) (layer "F.Cu") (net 2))
 (segment (start 117.8591 48.2173) (end 113.8335 48.2173) (width 0.25) (layer "F.Cu") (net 2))
 (segment (start 118.9465 49.3046) (end 119.1003 49.1508) (width 0.25) (layer "F.Cu") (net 2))
 (segment (start 119.1003 49.1508) (end 124.5133 49.1508) (width 0.25) (layer "F.Cu") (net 2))
 (segment (start 116.683 51.5681) (end 118.9465 49.3046) (width 0.25) (layer "F.Cu") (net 2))
 (segment (start 126.746 48.26) (end 125.4041 48.26) (width 0.25) (layer "F.Cu") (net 2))
 (segment (start 113.8335 48.2173) (end 112.4551 46.8389) (width 0.25) (layer "F.Cu") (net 2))
 (segment (start 112.4551 46.8389) (end 112.4551 45.085) (width 0.25) (layer "F.Cu") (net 2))
 (segment (start 113.632 45.085) (end 112.4551 45.085) (width 0.25) (layer "F.Cu") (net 2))
 (segment (start 111.4961 51.5681) (end 116.683 51.5681) (width 0.25) (layer "F.Cu") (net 2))
 (segment (start 109.358 48.9701) (end 111.7746 48.9701) (width 0.25) (layer "F.Cu") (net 3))
 (segment (start 113.8354 48.8611) (end 111.994 47.0197) (width 0.25) (layer "F.Cu") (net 3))
 (segment (start 115.5161 50.7139) (end 115.5161 49.3572) (width 0.25) (layer "F.Cu") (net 3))
 (segment (start 108.966 50.6778) (end 108.966 49.3621) (width 0.25) (layer "F.Cu") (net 3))
 (segment (start 111.7746 48.9701) (end 113.8955 51.091) (width 0.25) (layer "F.Cu") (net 3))
 (segment (start 113.632 43.815) (end 112.4551 43.815) (width 0.25) (layer "F.Cu") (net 3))
 (segment (start 107.8572 51.7866) (end 108.966 50.6778) (width 0.25) (layer "F.Cu") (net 3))
 (segment (start 126.746 45.72) (end 126.746 44.5281) (width 0.25) (layer "F.Cu") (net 3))
 (segment (start 94.504 50.292) (end 95.9986 51.7866) (width 0.25) (layer "F.Cu") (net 3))
 (segment (start 122.7454 44.5281) (end 122.3205 44.953) (width 0.25) (layer "F.Cu") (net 3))
 (segment (start 115.02 48.8611) (end 113.8354 48.8611) (width 0.25) (layer "F.Cu") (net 3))
 (segment (start 111.994 47.0197) (end 111.994 44.2761) (width 0.25) (layer "F.Cu") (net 3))
 (segment (start 126.746 44.5281) (end 122.7454 44.5281) (width 0.25) (layer "F.Cu") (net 3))
 (segment (start 122.3205 44.953) (end 115.9469 44.953) (width 0.25) (layer "F.Cu") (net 3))
 (segment (start 115.5161 49.3572) (end 115.02 48.8611) (width 0.25) (layer "F.Cu") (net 3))
 (segment (start 115.9469 44.953) (end 114.8089 43.815) (width 0.25) (layer "F.Cu") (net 3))
 (segment (start 113.632 43.815) (end 114.8089 43.815) (width 0.25) (layer "F.Cu") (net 3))
 (segment (start 113.8955 51.091) (end 115.139 51.091) (width 0.25) (layer "F.Cu") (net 3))
 (segment (start 95.9986 51.7866) (end 107.8572 51.7866) (width 0.25) (layer "F.Cu") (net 3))
 (segment (start 108.966 49.3621) (end 109.358 48.9701) (width 0.25) (layer "F.Cu") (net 3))
 (segment (start 111.994 44.2761) (end 112.4551 43.815) (width 0.25) (layer "F.Cu") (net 3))
 (segment (start 115.139 51.091) (end 115.5161 50.7139) (width 0.25) (layer "F.Cu") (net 3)))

